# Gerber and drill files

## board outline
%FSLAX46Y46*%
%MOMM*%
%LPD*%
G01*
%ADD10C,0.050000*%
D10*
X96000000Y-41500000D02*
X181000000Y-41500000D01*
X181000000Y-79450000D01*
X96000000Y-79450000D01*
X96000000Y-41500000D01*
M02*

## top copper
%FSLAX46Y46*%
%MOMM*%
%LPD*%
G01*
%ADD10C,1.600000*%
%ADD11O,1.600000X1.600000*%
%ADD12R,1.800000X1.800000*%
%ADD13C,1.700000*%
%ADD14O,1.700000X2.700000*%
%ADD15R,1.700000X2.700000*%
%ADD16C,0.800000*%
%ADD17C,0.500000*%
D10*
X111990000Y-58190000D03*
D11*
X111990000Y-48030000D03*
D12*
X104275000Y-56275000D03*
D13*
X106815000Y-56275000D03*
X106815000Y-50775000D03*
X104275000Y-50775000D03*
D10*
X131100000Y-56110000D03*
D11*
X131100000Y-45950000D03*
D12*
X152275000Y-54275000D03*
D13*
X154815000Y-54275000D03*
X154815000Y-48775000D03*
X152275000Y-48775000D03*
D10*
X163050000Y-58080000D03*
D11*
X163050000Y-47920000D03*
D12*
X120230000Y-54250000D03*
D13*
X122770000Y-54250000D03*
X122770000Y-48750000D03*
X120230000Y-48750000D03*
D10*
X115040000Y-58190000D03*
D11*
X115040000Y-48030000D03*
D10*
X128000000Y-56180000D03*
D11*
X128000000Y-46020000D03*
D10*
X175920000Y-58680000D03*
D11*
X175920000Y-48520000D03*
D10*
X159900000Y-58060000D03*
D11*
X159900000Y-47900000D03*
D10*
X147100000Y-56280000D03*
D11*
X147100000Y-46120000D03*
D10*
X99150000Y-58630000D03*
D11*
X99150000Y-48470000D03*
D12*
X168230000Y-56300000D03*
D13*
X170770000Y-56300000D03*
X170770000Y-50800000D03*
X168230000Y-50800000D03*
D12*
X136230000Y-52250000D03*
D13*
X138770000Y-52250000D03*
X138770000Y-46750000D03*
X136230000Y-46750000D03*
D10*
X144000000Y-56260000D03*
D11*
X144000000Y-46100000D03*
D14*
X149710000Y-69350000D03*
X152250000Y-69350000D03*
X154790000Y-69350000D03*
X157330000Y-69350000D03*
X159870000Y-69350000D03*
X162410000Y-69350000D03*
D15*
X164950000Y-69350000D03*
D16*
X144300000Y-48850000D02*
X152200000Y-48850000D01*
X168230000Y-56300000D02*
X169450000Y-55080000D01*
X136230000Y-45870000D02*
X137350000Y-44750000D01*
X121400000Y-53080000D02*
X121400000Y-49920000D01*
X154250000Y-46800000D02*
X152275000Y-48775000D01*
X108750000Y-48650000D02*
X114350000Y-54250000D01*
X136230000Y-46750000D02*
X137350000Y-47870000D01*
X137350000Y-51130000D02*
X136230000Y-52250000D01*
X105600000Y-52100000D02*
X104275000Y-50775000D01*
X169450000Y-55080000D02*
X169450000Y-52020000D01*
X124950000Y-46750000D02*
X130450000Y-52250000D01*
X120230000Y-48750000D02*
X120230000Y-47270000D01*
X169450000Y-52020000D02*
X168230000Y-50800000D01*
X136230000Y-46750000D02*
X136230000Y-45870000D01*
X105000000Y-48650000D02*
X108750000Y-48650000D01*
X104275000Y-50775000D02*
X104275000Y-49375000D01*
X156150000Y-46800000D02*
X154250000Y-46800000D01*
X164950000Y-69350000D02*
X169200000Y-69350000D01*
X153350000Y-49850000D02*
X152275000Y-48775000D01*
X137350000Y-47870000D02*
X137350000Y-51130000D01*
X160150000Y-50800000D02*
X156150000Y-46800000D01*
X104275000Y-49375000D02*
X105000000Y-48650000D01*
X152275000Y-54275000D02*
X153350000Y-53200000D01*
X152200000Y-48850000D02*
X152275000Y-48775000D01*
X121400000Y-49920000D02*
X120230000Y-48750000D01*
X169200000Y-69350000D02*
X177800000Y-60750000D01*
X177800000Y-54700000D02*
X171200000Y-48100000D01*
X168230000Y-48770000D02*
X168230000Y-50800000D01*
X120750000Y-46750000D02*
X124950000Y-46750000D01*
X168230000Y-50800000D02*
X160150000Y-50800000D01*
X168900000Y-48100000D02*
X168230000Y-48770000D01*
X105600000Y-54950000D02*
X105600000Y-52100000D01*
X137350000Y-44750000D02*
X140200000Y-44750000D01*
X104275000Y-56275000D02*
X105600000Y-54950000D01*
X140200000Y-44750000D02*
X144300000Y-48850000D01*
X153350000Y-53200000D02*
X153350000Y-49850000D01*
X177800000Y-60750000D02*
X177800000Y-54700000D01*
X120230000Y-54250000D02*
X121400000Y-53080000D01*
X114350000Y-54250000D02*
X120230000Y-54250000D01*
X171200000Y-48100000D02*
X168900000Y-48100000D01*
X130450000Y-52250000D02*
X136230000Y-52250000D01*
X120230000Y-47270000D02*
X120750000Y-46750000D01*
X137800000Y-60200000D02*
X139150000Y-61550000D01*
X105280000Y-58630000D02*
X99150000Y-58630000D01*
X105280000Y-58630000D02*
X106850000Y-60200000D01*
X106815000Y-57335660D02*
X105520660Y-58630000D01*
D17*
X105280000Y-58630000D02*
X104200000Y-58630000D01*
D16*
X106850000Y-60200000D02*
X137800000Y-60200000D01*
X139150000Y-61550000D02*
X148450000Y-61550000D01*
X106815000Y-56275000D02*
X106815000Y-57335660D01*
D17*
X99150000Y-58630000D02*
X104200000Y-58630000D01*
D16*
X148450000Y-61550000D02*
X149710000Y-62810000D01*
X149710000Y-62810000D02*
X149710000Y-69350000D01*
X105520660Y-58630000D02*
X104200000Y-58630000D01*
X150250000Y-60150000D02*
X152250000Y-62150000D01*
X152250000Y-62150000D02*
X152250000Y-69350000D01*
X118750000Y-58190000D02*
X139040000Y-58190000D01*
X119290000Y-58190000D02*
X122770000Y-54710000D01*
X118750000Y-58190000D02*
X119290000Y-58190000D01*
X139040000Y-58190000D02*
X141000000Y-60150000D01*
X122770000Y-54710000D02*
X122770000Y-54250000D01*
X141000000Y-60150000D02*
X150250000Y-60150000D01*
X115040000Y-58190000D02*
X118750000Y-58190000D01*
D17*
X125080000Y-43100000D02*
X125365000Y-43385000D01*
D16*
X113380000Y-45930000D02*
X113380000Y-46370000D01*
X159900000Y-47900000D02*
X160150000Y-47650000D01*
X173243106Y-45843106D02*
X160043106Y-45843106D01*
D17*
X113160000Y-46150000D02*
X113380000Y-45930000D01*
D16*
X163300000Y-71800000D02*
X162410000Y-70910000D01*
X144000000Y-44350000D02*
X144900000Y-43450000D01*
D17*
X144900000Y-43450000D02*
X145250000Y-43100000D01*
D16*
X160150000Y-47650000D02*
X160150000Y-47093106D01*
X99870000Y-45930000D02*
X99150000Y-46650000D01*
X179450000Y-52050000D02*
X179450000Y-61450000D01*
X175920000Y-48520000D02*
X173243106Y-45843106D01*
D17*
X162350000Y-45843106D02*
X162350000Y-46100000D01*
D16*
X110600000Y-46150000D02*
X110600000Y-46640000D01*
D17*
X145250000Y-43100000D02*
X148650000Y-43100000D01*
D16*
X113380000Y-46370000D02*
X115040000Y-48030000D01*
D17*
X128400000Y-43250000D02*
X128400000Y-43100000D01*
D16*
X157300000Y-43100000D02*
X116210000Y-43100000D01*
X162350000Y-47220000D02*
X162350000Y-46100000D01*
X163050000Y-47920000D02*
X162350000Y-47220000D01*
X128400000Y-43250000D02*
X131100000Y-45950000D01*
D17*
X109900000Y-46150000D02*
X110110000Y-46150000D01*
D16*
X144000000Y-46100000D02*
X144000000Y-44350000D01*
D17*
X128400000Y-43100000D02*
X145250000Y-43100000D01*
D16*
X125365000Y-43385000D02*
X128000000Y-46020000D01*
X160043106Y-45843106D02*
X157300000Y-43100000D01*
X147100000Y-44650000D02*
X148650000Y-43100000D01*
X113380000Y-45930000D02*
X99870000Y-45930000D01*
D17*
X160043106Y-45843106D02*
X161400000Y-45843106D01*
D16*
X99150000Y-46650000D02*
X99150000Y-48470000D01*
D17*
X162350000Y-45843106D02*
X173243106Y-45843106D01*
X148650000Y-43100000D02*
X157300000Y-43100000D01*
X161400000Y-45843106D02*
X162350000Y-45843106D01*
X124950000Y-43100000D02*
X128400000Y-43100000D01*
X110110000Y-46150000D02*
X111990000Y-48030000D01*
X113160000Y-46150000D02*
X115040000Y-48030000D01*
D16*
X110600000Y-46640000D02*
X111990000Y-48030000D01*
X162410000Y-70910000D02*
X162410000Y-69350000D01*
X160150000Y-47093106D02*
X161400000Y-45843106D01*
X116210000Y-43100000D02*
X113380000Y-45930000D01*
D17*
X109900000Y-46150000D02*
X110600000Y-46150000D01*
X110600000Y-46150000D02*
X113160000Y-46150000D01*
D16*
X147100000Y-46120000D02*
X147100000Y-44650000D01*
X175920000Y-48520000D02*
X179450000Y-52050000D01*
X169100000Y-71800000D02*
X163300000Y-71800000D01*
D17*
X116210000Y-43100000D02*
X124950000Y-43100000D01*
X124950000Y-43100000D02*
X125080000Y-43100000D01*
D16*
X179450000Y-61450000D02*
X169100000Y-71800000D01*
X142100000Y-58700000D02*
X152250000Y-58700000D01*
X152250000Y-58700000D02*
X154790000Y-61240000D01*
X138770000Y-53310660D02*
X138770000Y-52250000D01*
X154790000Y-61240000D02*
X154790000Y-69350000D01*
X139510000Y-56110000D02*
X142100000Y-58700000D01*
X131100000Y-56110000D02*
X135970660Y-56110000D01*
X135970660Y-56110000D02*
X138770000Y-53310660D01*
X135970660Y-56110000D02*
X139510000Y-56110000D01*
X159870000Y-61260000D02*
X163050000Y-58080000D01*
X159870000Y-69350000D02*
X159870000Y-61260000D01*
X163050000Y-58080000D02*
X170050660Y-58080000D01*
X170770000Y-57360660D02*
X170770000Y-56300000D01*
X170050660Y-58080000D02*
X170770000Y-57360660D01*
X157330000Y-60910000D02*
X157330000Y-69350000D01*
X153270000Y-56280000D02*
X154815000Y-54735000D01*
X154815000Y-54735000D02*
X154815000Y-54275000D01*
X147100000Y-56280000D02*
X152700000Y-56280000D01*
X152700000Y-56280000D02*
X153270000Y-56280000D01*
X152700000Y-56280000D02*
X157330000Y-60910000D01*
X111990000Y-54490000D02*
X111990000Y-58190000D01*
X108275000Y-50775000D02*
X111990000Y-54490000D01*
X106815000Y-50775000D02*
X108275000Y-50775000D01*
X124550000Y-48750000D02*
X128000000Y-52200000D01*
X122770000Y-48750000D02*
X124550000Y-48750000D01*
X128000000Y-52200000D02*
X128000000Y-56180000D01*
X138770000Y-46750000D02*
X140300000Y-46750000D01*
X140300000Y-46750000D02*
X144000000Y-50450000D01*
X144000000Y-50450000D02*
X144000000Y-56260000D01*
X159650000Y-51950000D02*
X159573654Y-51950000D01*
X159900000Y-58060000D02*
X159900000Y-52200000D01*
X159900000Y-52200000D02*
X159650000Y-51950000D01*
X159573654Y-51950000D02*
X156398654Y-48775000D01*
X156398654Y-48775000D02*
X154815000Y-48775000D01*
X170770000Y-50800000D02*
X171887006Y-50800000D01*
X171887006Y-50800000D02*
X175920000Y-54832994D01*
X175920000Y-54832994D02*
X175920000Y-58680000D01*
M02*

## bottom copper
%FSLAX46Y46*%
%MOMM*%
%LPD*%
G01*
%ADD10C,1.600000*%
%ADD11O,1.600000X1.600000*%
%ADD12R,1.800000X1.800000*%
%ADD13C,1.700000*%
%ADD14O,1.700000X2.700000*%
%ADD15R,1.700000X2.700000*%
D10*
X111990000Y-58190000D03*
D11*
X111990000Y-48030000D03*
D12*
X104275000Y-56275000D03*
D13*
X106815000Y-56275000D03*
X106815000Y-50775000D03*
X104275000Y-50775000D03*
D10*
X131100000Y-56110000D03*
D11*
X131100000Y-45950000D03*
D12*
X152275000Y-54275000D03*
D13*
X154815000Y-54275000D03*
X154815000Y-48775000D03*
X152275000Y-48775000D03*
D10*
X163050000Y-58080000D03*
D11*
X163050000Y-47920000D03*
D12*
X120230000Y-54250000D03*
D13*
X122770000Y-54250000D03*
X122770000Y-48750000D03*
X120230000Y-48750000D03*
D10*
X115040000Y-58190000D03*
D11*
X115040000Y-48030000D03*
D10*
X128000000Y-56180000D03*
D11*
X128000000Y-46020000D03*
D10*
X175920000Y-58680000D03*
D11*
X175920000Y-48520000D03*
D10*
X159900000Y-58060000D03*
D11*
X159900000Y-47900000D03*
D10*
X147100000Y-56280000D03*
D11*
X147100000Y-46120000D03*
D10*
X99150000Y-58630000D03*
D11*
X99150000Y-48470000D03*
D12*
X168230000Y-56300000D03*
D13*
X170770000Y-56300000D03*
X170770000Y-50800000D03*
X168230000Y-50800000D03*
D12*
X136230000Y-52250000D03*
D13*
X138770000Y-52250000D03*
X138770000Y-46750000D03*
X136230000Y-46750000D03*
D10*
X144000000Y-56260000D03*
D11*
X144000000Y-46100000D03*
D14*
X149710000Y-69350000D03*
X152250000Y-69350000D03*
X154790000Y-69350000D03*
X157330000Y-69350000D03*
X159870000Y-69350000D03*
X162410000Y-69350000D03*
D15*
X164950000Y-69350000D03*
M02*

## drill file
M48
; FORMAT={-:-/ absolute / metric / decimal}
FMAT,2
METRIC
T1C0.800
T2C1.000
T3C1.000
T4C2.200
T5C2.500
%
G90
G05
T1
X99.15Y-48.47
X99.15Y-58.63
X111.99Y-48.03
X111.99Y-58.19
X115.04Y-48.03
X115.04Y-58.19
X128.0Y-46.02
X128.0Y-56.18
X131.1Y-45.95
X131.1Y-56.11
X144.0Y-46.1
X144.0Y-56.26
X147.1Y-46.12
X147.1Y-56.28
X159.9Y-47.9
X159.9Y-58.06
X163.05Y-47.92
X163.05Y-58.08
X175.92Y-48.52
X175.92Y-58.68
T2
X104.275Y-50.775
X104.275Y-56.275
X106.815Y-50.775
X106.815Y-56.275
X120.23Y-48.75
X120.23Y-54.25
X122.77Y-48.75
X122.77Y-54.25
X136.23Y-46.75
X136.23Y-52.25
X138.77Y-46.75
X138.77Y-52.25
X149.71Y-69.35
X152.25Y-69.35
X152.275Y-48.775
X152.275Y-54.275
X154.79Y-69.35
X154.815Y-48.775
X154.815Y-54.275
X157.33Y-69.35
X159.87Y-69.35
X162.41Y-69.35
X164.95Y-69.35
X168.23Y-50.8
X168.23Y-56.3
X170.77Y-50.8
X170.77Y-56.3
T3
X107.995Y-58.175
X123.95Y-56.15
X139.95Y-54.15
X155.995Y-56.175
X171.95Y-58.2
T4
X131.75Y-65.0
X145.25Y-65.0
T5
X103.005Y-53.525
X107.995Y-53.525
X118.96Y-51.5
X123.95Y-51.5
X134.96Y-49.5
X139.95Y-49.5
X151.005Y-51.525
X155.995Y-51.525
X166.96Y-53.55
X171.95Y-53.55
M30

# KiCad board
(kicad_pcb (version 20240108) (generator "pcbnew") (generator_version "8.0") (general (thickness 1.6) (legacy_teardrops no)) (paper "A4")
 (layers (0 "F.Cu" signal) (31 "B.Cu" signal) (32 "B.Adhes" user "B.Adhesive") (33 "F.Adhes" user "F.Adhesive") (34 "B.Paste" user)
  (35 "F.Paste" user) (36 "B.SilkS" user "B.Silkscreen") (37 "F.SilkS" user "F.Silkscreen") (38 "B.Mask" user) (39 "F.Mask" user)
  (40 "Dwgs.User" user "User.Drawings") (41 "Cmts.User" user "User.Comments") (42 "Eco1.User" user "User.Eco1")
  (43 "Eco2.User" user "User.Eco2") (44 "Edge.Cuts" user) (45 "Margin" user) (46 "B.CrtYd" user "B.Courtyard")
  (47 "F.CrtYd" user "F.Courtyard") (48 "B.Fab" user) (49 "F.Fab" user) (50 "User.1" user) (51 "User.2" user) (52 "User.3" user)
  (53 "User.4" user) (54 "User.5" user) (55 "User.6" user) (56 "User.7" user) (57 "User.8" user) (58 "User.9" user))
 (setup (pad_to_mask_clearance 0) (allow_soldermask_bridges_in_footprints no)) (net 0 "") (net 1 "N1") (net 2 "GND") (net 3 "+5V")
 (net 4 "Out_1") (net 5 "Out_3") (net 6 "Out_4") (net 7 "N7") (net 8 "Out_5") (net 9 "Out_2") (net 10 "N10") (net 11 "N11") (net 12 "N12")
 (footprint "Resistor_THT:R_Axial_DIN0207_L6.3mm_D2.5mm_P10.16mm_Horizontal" (layer "F.Cu") (at 111.99 58.19 90)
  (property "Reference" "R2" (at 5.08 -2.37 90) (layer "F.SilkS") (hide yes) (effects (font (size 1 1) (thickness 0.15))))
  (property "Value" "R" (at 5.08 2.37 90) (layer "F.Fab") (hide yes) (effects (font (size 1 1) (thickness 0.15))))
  (pad "1" thru_hole circle (at 0 0 90) (size 1.6 1.6) (drill 0.8) (layers "*.Cu" "*.Mask") (remove_unused_layers no) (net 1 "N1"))
  (pad "2" thru_hole oval (at 10.16 0 90) (size 1.6 1.6) (drill 0.8) (layers "*.Cu" "*.Mask") (remove_unused_layers no) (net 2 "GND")))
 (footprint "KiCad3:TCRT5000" (layer "F.Cu") (at 105.545 53.525 90)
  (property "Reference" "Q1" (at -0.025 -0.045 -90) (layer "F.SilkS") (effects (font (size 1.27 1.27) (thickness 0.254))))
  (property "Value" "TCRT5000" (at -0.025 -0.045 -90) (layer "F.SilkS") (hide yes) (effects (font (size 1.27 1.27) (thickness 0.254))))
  (pad "" np_thru_hole circle (at -4.65 2.45 90) (size 1 1) (drill 1) (layers "*.Cu" "*.Mask"))
  (pad "" np_thru_hole circle (at 0 -2.54 90) (size 2.5 2.5) (drill 2.5) (layers "*.Cu" "*.Mask"))
  (pad "" np_thru_hole circle (at 0 2.45 90) (size 2.5 2.5) (drill 2.5) (layers "*.Cu" "*.Mask"))
  (pad "1" thru_hole rect (at -2.75 -1.27 90) (size 1.8 1.8) (drill 1) (layers "*.Cu" "*.Mask") (remove_unused_layers no) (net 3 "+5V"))
  (pad "2" thru_hole circle (at -2.75 1.27 90) (size 1.7 1.7) (drill 1) (layers "*.Cu" "*.Mask") (remove_unused_layers no) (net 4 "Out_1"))
  (pad "3" thru_hole circle (at 2.75 1.27 90) (size 1.7 1.7) (drill 1) (layers "*.Cu" "*.Mask") (remove_unused_layers no) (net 1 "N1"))
  (pad "4" thru_hole circle (at 2.75 -1.27 90) (size 1.7 1.7) (drill 1) (layers "*.Cu" "*.Mask") (remove_unused_layers no) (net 3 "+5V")))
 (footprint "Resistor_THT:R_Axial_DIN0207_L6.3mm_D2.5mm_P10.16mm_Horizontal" (layer "F.Cu") (at 131.1 56.11 90)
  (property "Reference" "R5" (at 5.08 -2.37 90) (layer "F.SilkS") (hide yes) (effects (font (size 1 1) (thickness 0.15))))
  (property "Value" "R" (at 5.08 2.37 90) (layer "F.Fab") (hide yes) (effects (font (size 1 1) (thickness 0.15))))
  (pad "1" thru_hole circle (at 0 0 90) (size 1.6 1.6) (drill 0.8) (layers "*.Cu" "*.Mask") (remove_unused_layers no) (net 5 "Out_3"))
  (pad "2" thru_hole oval (at 10.16 0 90) (size 1.6 1.6) (drill 0.8) (layers "*.Cu" "*.Mask") (remove_unused_layers no) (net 2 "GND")))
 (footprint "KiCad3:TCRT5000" (layer "F.Cu") (at 153.545 51.525 90)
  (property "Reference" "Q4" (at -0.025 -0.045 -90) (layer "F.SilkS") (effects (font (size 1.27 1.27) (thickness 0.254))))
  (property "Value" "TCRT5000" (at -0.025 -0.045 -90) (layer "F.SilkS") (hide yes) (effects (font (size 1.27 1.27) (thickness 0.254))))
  (pad "" np_thru_hole circle (at -4.65 2.45 90) (size 1 1) (drill 1) (layers "*.Cu" "*.Mask"))
  (pad "" np_thru_hole circle (at 0 -2.54 90) (size 2.5 2.5) (drill 2.5) (layers "*.Cu" "*.Mask"))
  (pad "" np_thru_hole circle (at 0 2.45 90) (size 2.5 2.5) (drill 2.5) (layers "*.Cu" "*.Mask"))
  (pad "1" thru_hole rect (at -2.75 -1.27 90) (size 1.8 1.8) (drill 1) (layers "*.Cu" "*.Mask") (remove_unused_layers no) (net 3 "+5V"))
  (pad "2" thru_hole circle (at -2.75 1.27 90) (size 1.7 1.7) (drill 1) (layers "*.Cu" "*.Mask") (remove_unused_layers no) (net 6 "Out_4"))
  (pad "3" thru_hole circle (at 2.75 1.27 90) (size 1.7 1.7) (drill 1) (layers "*.Cu" "*.Mask") (remove_unused_layers no) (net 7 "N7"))
  (pad "4" thru_hole circle (at 2.75 -1.27 90) (size 1.7 1.7) (drill 1) (layers "*.Cu" "*.Mask") (remove_unused_layers no) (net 3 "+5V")))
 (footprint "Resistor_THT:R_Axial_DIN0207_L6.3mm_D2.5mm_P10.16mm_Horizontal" (layer "F.Cu") (at 163.05 58.08 90)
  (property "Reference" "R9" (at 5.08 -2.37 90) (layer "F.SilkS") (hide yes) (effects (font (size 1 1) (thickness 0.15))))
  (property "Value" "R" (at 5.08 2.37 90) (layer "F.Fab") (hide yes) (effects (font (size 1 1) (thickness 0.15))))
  (pad "1" thru_hole circle (at 0 0 90) (size 1.6 1.6) (drill 0.8) (layers "*.Cu" "*.Mask") (remove_unused_layers no) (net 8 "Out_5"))
  (pad "2" thru_hole oval (at 10.16 0 90) (size 1.6 1.6) (drill 0.8) (layers "*.Cu" "*.Mask") (remove_unused_layers no) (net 2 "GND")))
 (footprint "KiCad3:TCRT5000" (layer "F.Cu") (at 121.5 51.5 90)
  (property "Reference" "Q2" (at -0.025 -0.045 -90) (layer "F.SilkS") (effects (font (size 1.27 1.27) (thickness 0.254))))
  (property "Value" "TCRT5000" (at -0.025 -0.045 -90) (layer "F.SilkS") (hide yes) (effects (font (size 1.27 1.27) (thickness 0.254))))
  (pad "" np_thru_hole circle (at -4.65 2.45 90) (size 1 1) (drill 1) (layers "*.Cu" "*.Mask"))
  (pad "" np_thru_hole circle (at 0 -2.54 90) (size 2.5 2.5) (drill 2.5) (layers "*.Cu" "*.Mask"))
  (pad "" np_thru_hole circle (at 0 2.45 90) (size 2.5 2.5) (drill 2.5) (layers "*.Cu" "*.Mask"))
  (pad "1" thru_hole rect (at -2.75 -1.27 90) (size 1.8 1.8) (drill 1) (layers "*.Cu" "*.Mask") (remove_unused_layers no) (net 3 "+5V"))
  (pad "2" thru_hole circle (at -2.75 1.27 90) (size 1.7 1.7) (drill 1) (layers "*.Cu" "*.Mask") (remove_unused_layers no) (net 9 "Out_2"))
  (pad "3" thru_hole circle (at 2.75 1.27 90) (size 1.7 1.7) (drill 1) (layers "*.Cu" "*.Mask") (remove_unused_layers no) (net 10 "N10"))
  (pad "4" thru_hole circle (at 2.75 -1.27 90) (size 1.7 1.7) (drill 1) (layers "*.Cu" "*.Mask") (remove_unused_layers no) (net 3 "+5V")))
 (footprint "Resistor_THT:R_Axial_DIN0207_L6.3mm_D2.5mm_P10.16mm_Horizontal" (layer "F.Cu") (at 115.04 58.19 90)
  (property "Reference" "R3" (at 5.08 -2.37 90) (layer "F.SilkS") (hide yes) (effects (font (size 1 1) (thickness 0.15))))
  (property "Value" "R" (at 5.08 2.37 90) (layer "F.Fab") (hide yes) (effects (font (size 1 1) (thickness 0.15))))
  (pad "1" thru_hole circle (at 0 0 90) (size 1.6 1.6) (drill 0.8) (layers "*.Cu" "*.Mask") (remove_unused_layers no) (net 9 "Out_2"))
  (pad "2" thru_hole oval (at 10.16 0 90) (size 1.6 1.6) (drill 0.8) (layers "*.Cu" "*.Mask") (remove_unused_layers no) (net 2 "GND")))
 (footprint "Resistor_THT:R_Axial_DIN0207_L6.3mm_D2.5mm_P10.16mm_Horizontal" (layer "F.Cu") (at 128 56.18 90)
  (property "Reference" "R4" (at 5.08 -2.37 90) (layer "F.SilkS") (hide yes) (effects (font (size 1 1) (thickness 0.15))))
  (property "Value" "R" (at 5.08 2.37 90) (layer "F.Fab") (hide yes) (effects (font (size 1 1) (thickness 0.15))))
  (pad "1" thru_hole circle (at 0 0 90) (size 1.6 1.6) (drill 0.8) (layers "*.Cu" "*.Mask") (remove_unused_layers no) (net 10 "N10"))
  (pad "2" thru_hole oval (at 10.16 0 90) (size 1.6 1.6) (drill 0.8) (layers "*.Cu" "*.Mask") (remove_unused_layers no) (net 2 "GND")))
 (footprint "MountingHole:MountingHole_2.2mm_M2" (layer "F.Cu") (at 131.75 65)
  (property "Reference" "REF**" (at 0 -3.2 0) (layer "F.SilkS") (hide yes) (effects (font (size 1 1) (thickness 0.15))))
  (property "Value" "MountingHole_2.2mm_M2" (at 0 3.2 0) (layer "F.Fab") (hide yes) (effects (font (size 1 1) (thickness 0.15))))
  (pad "" np_thru_hole circle (at 0 0) (size 2.2 2.2) (drill 2.2) (layers "*.Cu" "*.Mask")))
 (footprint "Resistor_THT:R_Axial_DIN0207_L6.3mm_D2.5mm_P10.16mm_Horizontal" (layer "F.Cu") (at 175.92 58.68 90)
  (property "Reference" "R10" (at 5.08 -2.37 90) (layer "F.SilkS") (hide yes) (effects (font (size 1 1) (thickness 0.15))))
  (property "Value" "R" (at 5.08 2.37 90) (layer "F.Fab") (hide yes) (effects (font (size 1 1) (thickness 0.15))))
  (pad "1" thru_hole circle (at 0 0 90) (size 1.6 1.6) (drill 0.8) (layers "*.Cu" "*.Mask") (remove_unused_layers no) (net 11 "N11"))
  (pad "2" thru_hole oval (at 10.16 0 90) (size 1.6 1.6) (drill 0.8) (layers "*.Cu" "*.Mask") (remove_unused_layers no) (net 2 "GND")))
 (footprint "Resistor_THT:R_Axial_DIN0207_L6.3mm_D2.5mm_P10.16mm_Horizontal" (layer "F.Cu") (at 159.9 58.06 90)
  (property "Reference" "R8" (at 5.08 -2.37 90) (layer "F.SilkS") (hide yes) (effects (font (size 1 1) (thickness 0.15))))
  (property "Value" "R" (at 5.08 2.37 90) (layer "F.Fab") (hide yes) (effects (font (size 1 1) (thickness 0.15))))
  (pad "1" thru_hole circle (at 0 0 90) (size 1.6 1.6) (drill 0.8) (layers "*.Cu" "*.Mask") (remove_unused_layers no) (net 7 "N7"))
  (pad "2" thru_hole oval (at 10.16 0 90) (size 1.6 1.6) (drill 0.8) (layers "*.Cu" "*.Mask") (remove_unused_layers no) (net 2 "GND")))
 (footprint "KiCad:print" (layer "F.Cu") (at 168.45 43.5)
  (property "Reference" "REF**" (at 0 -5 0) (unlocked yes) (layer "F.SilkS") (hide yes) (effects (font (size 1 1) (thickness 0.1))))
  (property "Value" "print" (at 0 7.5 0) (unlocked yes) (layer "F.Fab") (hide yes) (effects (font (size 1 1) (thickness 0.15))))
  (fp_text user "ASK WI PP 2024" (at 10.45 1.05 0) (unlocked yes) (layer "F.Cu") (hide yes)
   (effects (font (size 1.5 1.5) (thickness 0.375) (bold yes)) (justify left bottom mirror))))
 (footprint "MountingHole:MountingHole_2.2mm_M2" (layer "F.Cu") (at 145.25 65)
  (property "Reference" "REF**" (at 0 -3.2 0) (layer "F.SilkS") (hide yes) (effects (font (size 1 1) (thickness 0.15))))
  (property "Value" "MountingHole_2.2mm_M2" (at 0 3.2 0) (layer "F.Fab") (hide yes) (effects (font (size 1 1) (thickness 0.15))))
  (pad "" np_thru_hole circle (at 0 0) (size 2.2 2.2) (drill 2.2) (layers "*.Cu" "*.Mask")))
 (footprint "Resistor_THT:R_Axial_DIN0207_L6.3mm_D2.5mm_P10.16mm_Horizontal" (layer "F.Cu") (at 147.1 56.28 90)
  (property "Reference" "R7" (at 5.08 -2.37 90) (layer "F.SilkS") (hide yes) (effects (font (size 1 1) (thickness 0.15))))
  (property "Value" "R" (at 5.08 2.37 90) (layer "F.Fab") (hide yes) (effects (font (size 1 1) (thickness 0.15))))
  (pad "1" thru_hole circle (at 0 0 90) (size 1.6 1.6) (drill 0.8) (layers "*.Cu" "*.Mask") (remove_unused_layers no) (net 6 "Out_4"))
  (pad "2" thru_hole oval (at 10.16 0 90) (size 1.6 1.6) (drill 0.8) (layers "*.Cu" "*.Mask") (remove_unused_layers no) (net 2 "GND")))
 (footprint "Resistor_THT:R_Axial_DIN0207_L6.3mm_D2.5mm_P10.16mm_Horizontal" (layer "F.Cu") (at 99.15 58.63 90)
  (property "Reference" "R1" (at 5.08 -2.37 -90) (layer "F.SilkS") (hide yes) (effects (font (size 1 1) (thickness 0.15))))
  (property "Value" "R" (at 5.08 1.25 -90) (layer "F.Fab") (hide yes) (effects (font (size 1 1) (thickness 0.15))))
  (pad "1" thru_hole circle (at 0 0 90) (size 1.6 1.6) (drill 0.8) (layers "*.Cu" "*.Mask") (remove_unused_layers no) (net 4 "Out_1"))
  (pad "2" thru_hole oval (at 10.16 0 90) (size 1.6 1.6) (drill 0.8) (layers "*.Cu" "*.Mask") (remove_unused_layers no) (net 2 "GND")))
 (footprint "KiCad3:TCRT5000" (layer "F.Cu") (at 169.5 53.55 90)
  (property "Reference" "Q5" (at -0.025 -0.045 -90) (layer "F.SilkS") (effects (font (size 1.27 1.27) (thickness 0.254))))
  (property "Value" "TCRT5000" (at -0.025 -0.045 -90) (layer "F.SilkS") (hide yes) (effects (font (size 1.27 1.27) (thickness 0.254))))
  (pad "" np_thru_hole circle (at -4.65 2.45 90) (size 1 1) (drill 1) (layers "*.Cu" "*.Mask"))
  (pad "" np_thru_hole circle (at 0 -2.54 90) (size 2.5 2.5) (drill 2.5) (layers "*.Cu" "*.Mask"))
  (pad "" np_thru_hole circle (at 0 2.45 90) (size 2.5 2.5) (drill 2.5) (layers "*.Cu" "*.Mask"))
  (pad "1" thru_hole rect (at -2.75 -1.27 90) (size 1.8 1.8) (drill 1) (layers "*.Cu" "*.Mask") (remove_unused_layers no) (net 3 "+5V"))
  (pad "2" thru_hole circle (at -2.75 1.27 90) (size 1.7 1.7) (drill 1) (layers "*.Cu" "*.Mask") (remove_unused_layers no) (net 8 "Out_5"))
  (pad "3" thru_hole circle (at 2.75 1.27 90) (size 1.7 1.7) (drill 1) (layers "*.Cu" "*.Mask") (remove_unused_layers no) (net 11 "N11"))
  (pad "4" thru_hole circle (at 2.75 -1.27 90) (size 1.7 1.7) (drill 1) (layers "*.Cu" "*.Mask") (remove_unused_layers no) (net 3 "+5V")))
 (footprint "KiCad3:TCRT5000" (layer "F.Cu") (at 137.5 49.5 90)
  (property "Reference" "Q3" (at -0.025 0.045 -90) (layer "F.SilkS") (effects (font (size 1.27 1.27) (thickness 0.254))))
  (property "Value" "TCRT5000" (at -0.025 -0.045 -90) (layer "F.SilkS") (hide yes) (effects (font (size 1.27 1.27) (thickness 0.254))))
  (pad "" np_thru_hole circle (at -4.65 2.45 90) (size 1 1) (drill 1) (layers "*.Cu" "*.Mask"))
  (pad "" np_thru_hole circle (at 0 -2.54 90) (size 2.5 2.5) (drill 2.5) (layers "*.Cu" "*.Mask"))
  (pad "" np_thru_hole circle (at 0 2.45 90) (size 2.5 2.5) (drill 2.5) (layers "*.Cu" "*.Mask"))
  (pad "1" thru_hole rect (at -2.75 -1.27 90) (size 1.8 1.8) (drill 1) (layers "*.Cu" "*.Mask") (remove_unused_layers no) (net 3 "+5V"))
  (pad "2" thru_hole circle (at -2.75 1.27 90) (size 1.7 1.7) (drill 1) (layers "*.Cu" "*.Mask") (remove_unused_layers no) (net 5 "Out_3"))
  (pad "3" thru_hole circle (at 2.75 1.27 90) (size 1.7 1.7) (drill 1) (layers "*.Cu" "*.Mask") (remove_unused_layers no) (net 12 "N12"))
  (pad "4" thru_hole circle (at 2.75 -1.27 90) (size 1.7 1.7) (drill 1) (layers "*.Cu" "*.Mask") (remove_unused_layers no) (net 3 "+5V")))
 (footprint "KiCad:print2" (layer "F.Cu") (at 163.4 66.65)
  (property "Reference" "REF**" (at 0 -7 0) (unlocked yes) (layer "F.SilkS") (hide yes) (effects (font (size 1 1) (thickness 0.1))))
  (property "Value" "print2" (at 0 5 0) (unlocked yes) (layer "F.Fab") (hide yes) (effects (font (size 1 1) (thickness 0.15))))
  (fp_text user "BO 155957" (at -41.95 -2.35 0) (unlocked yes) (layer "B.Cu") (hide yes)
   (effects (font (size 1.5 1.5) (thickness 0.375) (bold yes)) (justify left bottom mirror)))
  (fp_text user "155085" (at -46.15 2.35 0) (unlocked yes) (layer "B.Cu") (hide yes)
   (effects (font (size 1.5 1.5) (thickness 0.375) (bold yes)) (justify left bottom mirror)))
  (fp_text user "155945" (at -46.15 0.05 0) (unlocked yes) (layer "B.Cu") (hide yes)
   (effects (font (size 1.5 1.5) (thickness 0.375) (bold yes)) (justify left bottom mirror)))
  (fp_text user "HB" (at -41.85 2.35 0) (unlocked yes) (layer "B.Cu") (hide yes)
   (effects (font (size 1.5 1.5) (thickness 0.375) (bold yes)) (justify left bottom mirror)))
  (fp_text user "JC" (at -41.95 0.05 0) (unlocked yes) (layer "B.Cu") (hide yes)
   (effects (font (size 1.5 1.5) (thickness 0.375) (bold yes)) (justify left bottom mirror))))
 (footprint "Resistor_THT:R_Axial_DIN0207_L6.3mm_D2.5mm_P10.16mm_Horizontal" (layer "F.Cu") (at 144 56.26 90)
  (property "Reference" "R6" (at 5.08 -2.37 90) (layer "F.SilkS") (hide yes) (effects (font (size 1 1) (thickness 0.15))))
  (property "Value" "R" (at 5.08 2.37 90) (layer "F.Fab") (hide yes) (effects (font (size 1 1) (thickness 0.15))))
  (pad "1" thru_hole circle (at 0 0 90) (size 1.6 1.6) (drill 0.8) (layers "*.Cu" "*.Mask") (remove_unused_layers no) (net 12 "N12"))
  (pad "2" thru_hole oval (at 10.16 0 90) (size 1.6 1.6) (drill 0.8) (layers "*.Cu" "*.Mask") (remove_unused_layers no) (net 2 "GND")))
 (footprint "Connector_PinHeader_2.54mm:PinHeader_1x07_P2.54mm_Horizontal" (layer "B.Cu") (at 149.71 69.35 -90)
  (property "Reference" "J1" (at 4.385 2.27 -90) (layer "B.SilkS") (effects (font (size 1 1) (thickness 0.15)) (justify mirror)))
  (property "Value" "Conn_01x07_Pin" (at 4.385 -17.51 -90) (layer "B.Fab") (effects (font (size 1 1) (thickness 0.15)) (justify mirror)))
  (pad "1" thru_hole oval (at 0 0 270) (size 2.7 1.7) (drill 1) (layers "*.Cu" "*.Mask") (remove_unused_layers no) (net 4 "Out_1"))
  (pad "2" thru_hole oval (at 0 -2.54 270) (size 2.7 1.7) (drill 1) (layers "*.Cu" "*.Mask") (remove_unused_layers no) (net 9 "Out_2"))
  (pad "3" thru_hole oval (at 0 -5.08 270) (size 2.7 1.7) (drill 1) (layers "*.Cu" "*.Mask") (remove_unused_layers no) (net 5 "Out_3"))
  (pad "4" thru_hole oval (at 0 -7.62 270) (size 2.7 1.7) (drill 1) (layers "*.Cu" "*.Mask") (remove_unused_layers no) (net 6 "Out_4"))
  (pad "5" thru_hole oval (at 0 -10.16 270) (size 2.7 1.7) (drill 1) (layers "*.Cu" "*.Mask") (remove_unused_layers no) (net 8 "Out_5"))
  (pad "6" thru_hole oval (at 0 -12.7 270) (size 2.7 1.7) (drill 1) (layers "*.Cu" "*.Mask") (remove_unused_layers no) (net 2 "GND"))
  (pad "7" thru_hole rect (at 0 -15.24 270) (size 2.7 1.7) (drill 1) (layers "*.Cu" "*.Mask") (remove_unused_layers no) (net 3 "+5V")))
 (gr_rect (start 96 41.5) (end 181 79.45) (stroke (width 0.05) (type default)) (fill none) (layer "Edge.Cuts"))
 (segment (start 144.3 48.85) (end 152.2 48.85) (width 0.8) (layer "F.Cu") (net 3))
 (segment (start 168.23 56.3) (end 169.45 55.08) (width 0.8) (layer "F.Cu") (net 3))
 (segment (start 136.23 45.87) (end 137.35 44.75) (width 0.8) (layer "F.Cu") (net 3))
 (segment (start 121.4 53.08) (end 121.4 49.92) (width 0.8) (layer "F.Cu") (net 3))
 (segment (start 154.25 46.8) (end 152.275 48.775) (width 0.8) (layer "F.Cu") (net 3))
 (segment (start 108.75 48.65) (end 114.35 54.25) (width 0.8) (layer "F.Cu") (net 3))
 (segment (start 136.23 46.75) (end 137.35 47.87) (width 0.8) (layer "F.Cu") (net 3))
 (segment (start 137.35 51.13) (end 136.23 52.25) (width 0.8) (layer "F.Cu") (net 3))
 (segment (start 105.6 52.1) (end 104.275 50.775) (width 0.8) (layer "F.Cu") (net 3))
 (segment (start 169.45 55.08) (end 169.45 52.02) (width 0.8) (layer "F.Cu") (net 3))
 (segment (start 124.95 46.75) (end 130.45 52.25) (width 0.8) (layer "F.Cu") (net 3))
 (segment (start 120.23 48.75) (end 120.23 47.27) (width 0.8) (layer "F.Cu") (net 3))
 (segment (start 169.45 52.02) (end 168.23 50.8) (width 0.8) (layer "F.Cu") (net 3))
 (segment (start 136.23 46.75) (end 136.23 45.87) (width 0.8) (layer "F.Cu") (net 3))
 (segment (start 105 48.65) (end 108.75 48.65) (width 0.8) (layer "F.Cu") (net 3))
 (segment (start 104.275 50.775) (end 104.275 49.375) (width 0.8) (layer "F.Cu") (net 3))
 (segment (start 156.15 46.8) (end 154.25 46.8) (width 0.8) (layer "F.Cu") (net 3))
 (segment (start 164.95 69.35) (end 169.2 69.35) (width 0.8) (layer "F.Cu") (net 3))
 (segment (start 153.35 49.85) (end 152.275 48.775) (width 0.8) (layer "F.Cu") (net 3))
 (segment (start 137.35 47.87) (end 137.35 51.13) (width 0.8) (layer "F.Cu") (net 3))
 (segment (start 160.15 50.8) (end 156.15 46.8) (width 0.8) (layer "F.Cu") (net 3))
 (segment (start 104.275 49.375) (end 105 48.65) (width 0.8) (layer "F.Cu") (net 3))
 (segment (start 152.275 54.275) (end 153.35 53.2) (width 0.8) (layer "F.Cu") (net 3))
 (segment (start 152.2 48.85) (end 152.275 48.775) (width 0.8) (layer "F.Cu") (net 3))
 (segment (start 121.4 49.92) (end 120.23 48.75) (width 0.8) (layer "F.Cu") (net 3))
 (segment (start 169.2 69.35) (end 177.8 60.75) (width 0.8) (layer "F.Cu") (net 3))
 (segment (start 177.8 54.7) (end 171.2 48.1) (width 0.8) (layer "F.Cu") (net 3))
 (segment (start 168.23 48.77) (end 168.23 50.8) (width 0.8) (layer "F.Cu") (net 3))
 (segment (start 120.75 46.75) (end 124.95 46.75) (width 0.8) (layer "F.Cu") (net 3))
 (segment (start 168.23 50.8) (end 160.15 50.8) (width 0.8) (layer "F.Cu") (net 3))
 (segment (start 168.9 48.1) (end 168.23 48.77) (width 0.8) (layer "F.Cu") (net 3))
 (segment (start 105.6 54.95) (end 105.6 52.1) (width 0.8) (layer "F.Cu") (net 3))
 (segment (start 137.35 44.75) (end 140.2 44.75) (width 0.8) (layer "F.Cu") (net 3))
 (segment (start 104.275 56.275) (end 105.6 54.95) (width 0.8) (layer "F.Cu") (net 3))
 (segment (start 140.2 44.75) (end 144.3 48.85) (width 0.8) (layer "F.Cu") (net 3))
 (segment (start 153.35 53.2) (end 153.35 49.85) (width 0.8) (layer "F.Cu") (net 3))
 (segment (start 177.8 60.75) (end 177.8 54.7) (width 0.8) (layer "F.Cu") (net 3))
 (segment (start 120.23 54.25) (end 121.4 53.08) (width 0.8) (layer "F.Cu") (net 3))
 (segment (start 114.35 54.25) (end 120.23 54.25) (width 0.8) (layer "F.Cu") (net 3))
 (segment (start 171.2 48.1) (end 168.9 48.1) (width 0.8) (layer "F.Cu") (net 3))
 (segment (start 130.45 52.25) (end 136.23 52.25) (width 0.8) (layer "F.Cu") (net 3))
 (segment (start 120.23 47.27) (end 120.75 46.75) (width 0.8) (layer "F.Cu") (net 3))
 (segment (start 137.8 60.2) (end 139.15 61.55) (width 0.8) (layer "F.Cu") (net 4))
 (segment (start 105.28 58.63) (end 99.15 58.63) (width 0.8) (layer "F.Cu") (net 4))
 (segment (start 105.28 58.63) (end 106.85 60.2) (width 0.8) (layer "F.Cu") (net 4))
 (segment (start 106.815 57.33566) (end 105.52066 58.63) (width 0.8) (layer "F.Cu") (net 4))
 (segment (start 105.28 58.63) (end 104.2 58.63) (width 0.5) (layer "F.Cu") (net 4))
 (segment (start 106.85 60.2) (end 137.8 60.2) (width 0.8) (layer "F.Cu") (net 4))
 (segment (start 139.15 61.55) (end 148.45 61.55) (width 0.8) (layer "F.Cu") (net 4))
 (segment (start 106.815 56.275) (end 106.815 57.33566) (width 0.8) (layer "F.Cu") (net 4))
 (segment (start 99.15 58.63) (end 104.2 58.63) (width 0.5) (layer "F.Cu") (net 4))
 (segment (start 148.45 61.55) (end 149.71 62.81) (width 0.8) (layer "F.Cu") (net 4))
 (segment (start 149.71 62.81) (end 149.71 69.35) (width 0.8) (layer "F.Cu") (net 4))
 (segment (start 105.52066 58.63) (end 104.2 58.63) (width 0.8) (layer "F.Cu") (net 4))
 (segment (start 150.25 60.15) (end 152.25 62.15) (width 0.8) (layer "F.Cu") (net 9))
 (segment (start 152.25 62.15) (end 152.25 69.35) (width 0.8) (layer "F.Cu") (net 9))
 (segment (start 118.75 58.19) (end 139.04 58.19) (width 0.8) (layer "F.Cu") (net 9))
 (segment (start 119.29 58.19) (end 122.77 54.71) (width 0.8) (layer "F.Cu") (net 9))
 (segment (start 118.75 58.19) (end 119.29 58.19) (width 0.8) (layer "F.Cu") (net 9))
 (segment (start 139.04 58.19) (end 141 60.15) (width 0.8) (layer "F.Cu") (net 9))
 (segment (start 122.77 54.71) (end 122.77 54.25) (width 0.8) (layer "F.Cu") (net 9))
 (segment (start 141 60.15) (end 150.25 60.15) (width 0.8) (layer "F.Cu") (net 9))
 (segment (start 115.04 58.19) (end 118.75 58.19) (width 0.8) (layer "F.Cu") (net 9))
 (segment (start 125.08 43.1) (end 125.365 43.385) (width 0.5) (layer "F.Cu") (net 2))
 (segment (start 113.38 45.93) (end 113.38 46.37) (width 0.8) (layer "F.Cu") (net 2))
 (segment (start 159.9 47.9) (end 160.15 47.65) (width 0.8) (layer "F.Cu") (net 2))
 (segment (start 173.243106 45.843106) (end 160.043106 45.843106) (width 0.8) (layer "F.Cu") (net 2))
 (segment (start 113.16 46.15) (end 113.38 45.93) (width 0.5) (layer "F.Cu") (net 2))
 (segment (start 163.3 71.8) (end 162.41 70.91) (width 0.8) (layer "F.Cu") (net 2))
 (segment (start 144 44.35) (end 144.9 43.45) (width 0.8) (layer "F.Cu") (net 2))
 (segment (start 144.9 43.45) (end 145.25 43.1) (width 0.5) (layer "F.Cu") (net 2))
 (segment (start 160.15 47.65) (end 160.15 47.093106) (width 0.8) (layer "F.Cu") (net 2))
 (segment (start 99.87 45.93) (end 99.15 46.65) (width 0.8) (layer "F.Cu") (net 2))
 (segment (start 179.45 52.05) (end 179.45 61.45) (width 0.8) (layer "F.Cu") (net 2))
 (segment (start 175.92 48.52) (end 173.243106 45.843106) (width 0.8) (layer "F.Cu") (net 2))
 (segment (start 162.35 45.843106) (end 162.35 46.1) (width 0.5) (layer "F.Cu") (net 2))
 (segment (start 110.6 46.15) (end 110.6 46.64) (width 0.8) (layer "F.Cu") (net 2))
 (segment (start 145.25 43.1) (end 148.65 43.1) (width 0.5) (layer "F.Cu") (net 2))
 (segment (start 113.38 46.37) (end 115.04 48.03) (width 0.8) (layer "F.Cu") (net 2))
 (segment (start 128.4 43.25) (end 128.4 43.1) (width 0.5) (layer "F.Cu") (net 2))
 (segment (start 157.3 43.1) (end 116.21 43.1) (width 0.8) (layer "F.Cu") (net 2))
 (segment (start 162.35 47.22) (end 162.35 46.1) (width 0.8) (layer "F.Cu") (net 2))
 (segment (start 163.05 47.92) (end 162.35 47.22) (width 0.8) (layer "F.Cu") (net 2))
 (segment (start 128.4 43.25) (end 131.1 45.95) (width 0.8) (layer "F.Cu") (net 2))
 (segment (start 109.9 46.15) (end 110.11 46.15) (width 0.5) (layer "F.Cu") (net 2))
 (segment (start 144 46.1) (end 144 44.35) (width 0.8) (layer "F.Cu") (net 2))
 (segment (start 128.4 43.1) (end 145.25 43.1) (width 0.5) (layer "F.Cu") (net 2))
 (segment (start 125.365 43.385) (end 128 46.02) (width 0.8) (layer "F.Cu") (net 2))
 (segment (start 160.043106 45.843106) (end 157.3 43.1) (width 0.8) (layer "F.Cu") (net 2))
 (segment (start 147.1 44.65) (end 148.65 43.1) (width 0.8) (layer "F.Cu") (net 2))
 (segment (start 113.38 45.93) (end 99.87 45.93) (width 0.8) (layer "F.Cu") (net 2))
 (segment (start 160.043106 45.843106) (end 161.4 45.843106) (width 0.5) (layer "F.Cu") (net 2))
 (segment (start 99.15 46.65) (end 99.15 48.47) (width 0.8) (layer "F.Cu") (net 2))
 (segment (start 162.35 45.843106) (end 173.243106 45.843106) (width 0.5) (layer "F.Cu") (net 2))
 (segment (start 148.65 43.1) (end 157.3 43.1) (width 0.5) (layer "F.Cu") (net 2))
 (segment (start 161.4 45.843106) (end 162.35 45.843106) (width 0.5) (layer "F.Cu") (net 2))
 (segment (start 124.95 43.1) (end 128.4 43.1) (width 0.5) (layer "F.Cu") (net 2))
 (segment (start 110.11 46.15) (end 111.99 48.03) (width 0.5) (layer "F.Cu") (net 2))
 (segment (start 113.16 46.15) (end 115.04 48.03) (width 0.5) (layer "F.Cu") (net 2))
 (segment (start 110.6 46.64) (end 111.99 48.03) (width 0.8) (layer "F.Cu") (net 2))
 (segment (start 162.41 70.91) (end 162.41 69.35) (width 0.8) (layer "F.Cu") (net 2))
 (segment (start 160.15 47.093106) (end 161.4 45.843106) (width 0.8) (layer "F.Cu") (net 2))
 (segment (start 116.21 43.1) (end 113.38 45.93) (width 0.8) (layer "F.Cu") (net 2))
 (segment (start 109.9 46.15) (end 110.6 46.15) (width 0.5) (layer "F.Cu") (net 2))
 (segment (start 110.6 46.15) (end 113.16 46.15) (width 0.5) (layer "F.Cu") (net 2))
 (segment (start 147.1 46.12) (end 147.1 44.65) (width 0.8) (layer "F.Cu") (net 2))
 (segment (start 175.92 48.52) (end 179.45 52.05) (width 0.8) (layer "F.Cu") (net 2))
 (segment (start 169.1 71.8) (end 163.3 71.8) (width 0.8) (layer "F.Cu") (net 2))
 (segment (start 116.21 43.1) (end 124.95 43.1) (width 0.5) (layer "F.Cu") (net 2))
 (segment (start 124.95 43.1) (end 125.08 43.1) (width 0.5) (layer "F.Cu") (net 2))
 (segment (start 179.45 61.45) (end 169.1 71.8) (width 0.8) (layer "F.Cu") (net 2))
 (segment (start 142.1 58.7) (end 152.25 58.7) (width 0.8) (layer "F.Cu") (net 5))
 (segment (start 152.25 58.7) (end 154.79 61.24) (width 0.8) (layer "F.Cu") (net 5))
 (segment (start 138.77 53.31066) (end 138.77 52.25) (width 0.8) (layer "F.Cu") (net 5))
 (segment (start 154.79 61.24) (end 154.79 69.35) (width 0.8) (layer "F.Cu") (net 5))
 (segment (start 139.51 56.11) (end 142.1 58.7) (width 0.8) (layer "F.Cu") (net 5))
 (segment (start 131.1 56.11) (end 135.97066 56.11) (width 0.8) (layer "F.Cu") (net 5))
 (segment (start 135.97066 56.11) (end 138.77 53.31066) (width 0.8) (layer "F.Cu") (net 5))
 (segment (start 135.97066 56.11) (end 139.51 56.11) (width 0.8) (layer "F.Cu") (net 5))
 (segment (start 159.87 61.26) (end 163.05 58.08) (width 0.8) (layer "F.Cu") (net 8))
 (segment (start 159.87 69.35) (end 159.87 61.26) (width 0.8) (layer "F.Cu") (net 8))
 (segment (start 163.05 58.08) (end 170.05066 58.08) (width 0.8) (layer "F.Cu") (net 8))
 (segment (start 170.77 57.36066) (end 170.77 56.3) (width 0.8) (layer "F.Cu") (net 8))
 (segment (start 170.05066 58.08) (end 170.77 57.36066) (width 0.8) (layer "F.Cu") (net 8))
 (segment (start 157.33 60.91) (end 157.33 69.35) (width 0.8) (layer "F.Cu") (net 6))
 (segment (start 153.27 56.28) (end 154.815 54.735) (width 0.8) (layer "F.Cu") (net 6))
 (segment (start 154.815 54.735) (end 154.815 54.275) (width 0.8) (layer "F.Cu") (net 6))
 (segment (start 147.1 56.28) (end 152.7 56.28) (width 0.8) (layer "F.Cu") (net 6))
 (segment (start 152.7 56.28) (end 153.27 56.28) (width 0.8) (layer "F.Cu") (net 6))
 (segment (start 152.7 56.28) (end 157.33 60.91) (width 0.8) (layer "F.Cu") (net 6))
 (segment (start 111.99 54.49) (end 111.99 58.19) (width 0.8) (layer "F.Cu") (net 1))
 (segment (start 108.275 50.775) (end 111.99 54.49) (width 0.8) (layer "F.Cu") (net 1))
 (segment (start 106.815 50.775) (end 108.275 50.775) (width 0.8) (layer "F.Cu") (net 1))
 (segment (start 124.55 48.75) (end 128 52.2) (width 0.8) (layer "F.Cu") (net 10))
 (segment (start 122.77 48.75) (end 124.55 48.75) (width 0.8) (layer "F.Cu") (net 10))
 (segment (start 128 52.2) (end 128 56.18) (width 0.8) (layer "F.Cu") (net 10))
 (segment (start 138.77 46.75) (end 140.3 46.75) (width 0.8) (layer "F.Cu") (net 12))
 (segment (start 140.3 46.75) (end 144 50.45) (width 0.8) (layer "F.Cu") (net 12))
 (segment (start 144 50.45) (end 144 56.26) (width 0.8) (layer "F.Cu") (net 12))
 (segment (start 159.65 51.95) (end 159.573654 51.95) (width 0.8) (layer "F.Cu") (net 7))
 (segment (start 159.9 58.06) (end 159.9 52.2) (width 0.8) (layer "F.Cu") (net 7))
 (segment (start 159.9 52.2) (end 159.65 51.95) (width 0.8) (layer "F.Cu") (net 7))
 (segment (start 159.573654 51.95) (end 156.398654 48.775) (width 0.8) (layer "F.Cu") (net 7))
 (segment (start 156.398654 48.775) (end 154.815 48.775) (width 0.8) (layer "F.Cu") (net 7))
 (segment (start 170.77 50.8) (end 171.887006 50.8) (width 0.8) (layer "F.Cu") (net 11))
 (segment (start 171.887006 50.8) (end 175.92 54.832994) (width 0.8) (layer "F.Cu") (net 11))
 (segment (start 175.92 54.832994) (end 175.92 58.68) (width 0.8) (layer "F.Cu") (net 11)))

